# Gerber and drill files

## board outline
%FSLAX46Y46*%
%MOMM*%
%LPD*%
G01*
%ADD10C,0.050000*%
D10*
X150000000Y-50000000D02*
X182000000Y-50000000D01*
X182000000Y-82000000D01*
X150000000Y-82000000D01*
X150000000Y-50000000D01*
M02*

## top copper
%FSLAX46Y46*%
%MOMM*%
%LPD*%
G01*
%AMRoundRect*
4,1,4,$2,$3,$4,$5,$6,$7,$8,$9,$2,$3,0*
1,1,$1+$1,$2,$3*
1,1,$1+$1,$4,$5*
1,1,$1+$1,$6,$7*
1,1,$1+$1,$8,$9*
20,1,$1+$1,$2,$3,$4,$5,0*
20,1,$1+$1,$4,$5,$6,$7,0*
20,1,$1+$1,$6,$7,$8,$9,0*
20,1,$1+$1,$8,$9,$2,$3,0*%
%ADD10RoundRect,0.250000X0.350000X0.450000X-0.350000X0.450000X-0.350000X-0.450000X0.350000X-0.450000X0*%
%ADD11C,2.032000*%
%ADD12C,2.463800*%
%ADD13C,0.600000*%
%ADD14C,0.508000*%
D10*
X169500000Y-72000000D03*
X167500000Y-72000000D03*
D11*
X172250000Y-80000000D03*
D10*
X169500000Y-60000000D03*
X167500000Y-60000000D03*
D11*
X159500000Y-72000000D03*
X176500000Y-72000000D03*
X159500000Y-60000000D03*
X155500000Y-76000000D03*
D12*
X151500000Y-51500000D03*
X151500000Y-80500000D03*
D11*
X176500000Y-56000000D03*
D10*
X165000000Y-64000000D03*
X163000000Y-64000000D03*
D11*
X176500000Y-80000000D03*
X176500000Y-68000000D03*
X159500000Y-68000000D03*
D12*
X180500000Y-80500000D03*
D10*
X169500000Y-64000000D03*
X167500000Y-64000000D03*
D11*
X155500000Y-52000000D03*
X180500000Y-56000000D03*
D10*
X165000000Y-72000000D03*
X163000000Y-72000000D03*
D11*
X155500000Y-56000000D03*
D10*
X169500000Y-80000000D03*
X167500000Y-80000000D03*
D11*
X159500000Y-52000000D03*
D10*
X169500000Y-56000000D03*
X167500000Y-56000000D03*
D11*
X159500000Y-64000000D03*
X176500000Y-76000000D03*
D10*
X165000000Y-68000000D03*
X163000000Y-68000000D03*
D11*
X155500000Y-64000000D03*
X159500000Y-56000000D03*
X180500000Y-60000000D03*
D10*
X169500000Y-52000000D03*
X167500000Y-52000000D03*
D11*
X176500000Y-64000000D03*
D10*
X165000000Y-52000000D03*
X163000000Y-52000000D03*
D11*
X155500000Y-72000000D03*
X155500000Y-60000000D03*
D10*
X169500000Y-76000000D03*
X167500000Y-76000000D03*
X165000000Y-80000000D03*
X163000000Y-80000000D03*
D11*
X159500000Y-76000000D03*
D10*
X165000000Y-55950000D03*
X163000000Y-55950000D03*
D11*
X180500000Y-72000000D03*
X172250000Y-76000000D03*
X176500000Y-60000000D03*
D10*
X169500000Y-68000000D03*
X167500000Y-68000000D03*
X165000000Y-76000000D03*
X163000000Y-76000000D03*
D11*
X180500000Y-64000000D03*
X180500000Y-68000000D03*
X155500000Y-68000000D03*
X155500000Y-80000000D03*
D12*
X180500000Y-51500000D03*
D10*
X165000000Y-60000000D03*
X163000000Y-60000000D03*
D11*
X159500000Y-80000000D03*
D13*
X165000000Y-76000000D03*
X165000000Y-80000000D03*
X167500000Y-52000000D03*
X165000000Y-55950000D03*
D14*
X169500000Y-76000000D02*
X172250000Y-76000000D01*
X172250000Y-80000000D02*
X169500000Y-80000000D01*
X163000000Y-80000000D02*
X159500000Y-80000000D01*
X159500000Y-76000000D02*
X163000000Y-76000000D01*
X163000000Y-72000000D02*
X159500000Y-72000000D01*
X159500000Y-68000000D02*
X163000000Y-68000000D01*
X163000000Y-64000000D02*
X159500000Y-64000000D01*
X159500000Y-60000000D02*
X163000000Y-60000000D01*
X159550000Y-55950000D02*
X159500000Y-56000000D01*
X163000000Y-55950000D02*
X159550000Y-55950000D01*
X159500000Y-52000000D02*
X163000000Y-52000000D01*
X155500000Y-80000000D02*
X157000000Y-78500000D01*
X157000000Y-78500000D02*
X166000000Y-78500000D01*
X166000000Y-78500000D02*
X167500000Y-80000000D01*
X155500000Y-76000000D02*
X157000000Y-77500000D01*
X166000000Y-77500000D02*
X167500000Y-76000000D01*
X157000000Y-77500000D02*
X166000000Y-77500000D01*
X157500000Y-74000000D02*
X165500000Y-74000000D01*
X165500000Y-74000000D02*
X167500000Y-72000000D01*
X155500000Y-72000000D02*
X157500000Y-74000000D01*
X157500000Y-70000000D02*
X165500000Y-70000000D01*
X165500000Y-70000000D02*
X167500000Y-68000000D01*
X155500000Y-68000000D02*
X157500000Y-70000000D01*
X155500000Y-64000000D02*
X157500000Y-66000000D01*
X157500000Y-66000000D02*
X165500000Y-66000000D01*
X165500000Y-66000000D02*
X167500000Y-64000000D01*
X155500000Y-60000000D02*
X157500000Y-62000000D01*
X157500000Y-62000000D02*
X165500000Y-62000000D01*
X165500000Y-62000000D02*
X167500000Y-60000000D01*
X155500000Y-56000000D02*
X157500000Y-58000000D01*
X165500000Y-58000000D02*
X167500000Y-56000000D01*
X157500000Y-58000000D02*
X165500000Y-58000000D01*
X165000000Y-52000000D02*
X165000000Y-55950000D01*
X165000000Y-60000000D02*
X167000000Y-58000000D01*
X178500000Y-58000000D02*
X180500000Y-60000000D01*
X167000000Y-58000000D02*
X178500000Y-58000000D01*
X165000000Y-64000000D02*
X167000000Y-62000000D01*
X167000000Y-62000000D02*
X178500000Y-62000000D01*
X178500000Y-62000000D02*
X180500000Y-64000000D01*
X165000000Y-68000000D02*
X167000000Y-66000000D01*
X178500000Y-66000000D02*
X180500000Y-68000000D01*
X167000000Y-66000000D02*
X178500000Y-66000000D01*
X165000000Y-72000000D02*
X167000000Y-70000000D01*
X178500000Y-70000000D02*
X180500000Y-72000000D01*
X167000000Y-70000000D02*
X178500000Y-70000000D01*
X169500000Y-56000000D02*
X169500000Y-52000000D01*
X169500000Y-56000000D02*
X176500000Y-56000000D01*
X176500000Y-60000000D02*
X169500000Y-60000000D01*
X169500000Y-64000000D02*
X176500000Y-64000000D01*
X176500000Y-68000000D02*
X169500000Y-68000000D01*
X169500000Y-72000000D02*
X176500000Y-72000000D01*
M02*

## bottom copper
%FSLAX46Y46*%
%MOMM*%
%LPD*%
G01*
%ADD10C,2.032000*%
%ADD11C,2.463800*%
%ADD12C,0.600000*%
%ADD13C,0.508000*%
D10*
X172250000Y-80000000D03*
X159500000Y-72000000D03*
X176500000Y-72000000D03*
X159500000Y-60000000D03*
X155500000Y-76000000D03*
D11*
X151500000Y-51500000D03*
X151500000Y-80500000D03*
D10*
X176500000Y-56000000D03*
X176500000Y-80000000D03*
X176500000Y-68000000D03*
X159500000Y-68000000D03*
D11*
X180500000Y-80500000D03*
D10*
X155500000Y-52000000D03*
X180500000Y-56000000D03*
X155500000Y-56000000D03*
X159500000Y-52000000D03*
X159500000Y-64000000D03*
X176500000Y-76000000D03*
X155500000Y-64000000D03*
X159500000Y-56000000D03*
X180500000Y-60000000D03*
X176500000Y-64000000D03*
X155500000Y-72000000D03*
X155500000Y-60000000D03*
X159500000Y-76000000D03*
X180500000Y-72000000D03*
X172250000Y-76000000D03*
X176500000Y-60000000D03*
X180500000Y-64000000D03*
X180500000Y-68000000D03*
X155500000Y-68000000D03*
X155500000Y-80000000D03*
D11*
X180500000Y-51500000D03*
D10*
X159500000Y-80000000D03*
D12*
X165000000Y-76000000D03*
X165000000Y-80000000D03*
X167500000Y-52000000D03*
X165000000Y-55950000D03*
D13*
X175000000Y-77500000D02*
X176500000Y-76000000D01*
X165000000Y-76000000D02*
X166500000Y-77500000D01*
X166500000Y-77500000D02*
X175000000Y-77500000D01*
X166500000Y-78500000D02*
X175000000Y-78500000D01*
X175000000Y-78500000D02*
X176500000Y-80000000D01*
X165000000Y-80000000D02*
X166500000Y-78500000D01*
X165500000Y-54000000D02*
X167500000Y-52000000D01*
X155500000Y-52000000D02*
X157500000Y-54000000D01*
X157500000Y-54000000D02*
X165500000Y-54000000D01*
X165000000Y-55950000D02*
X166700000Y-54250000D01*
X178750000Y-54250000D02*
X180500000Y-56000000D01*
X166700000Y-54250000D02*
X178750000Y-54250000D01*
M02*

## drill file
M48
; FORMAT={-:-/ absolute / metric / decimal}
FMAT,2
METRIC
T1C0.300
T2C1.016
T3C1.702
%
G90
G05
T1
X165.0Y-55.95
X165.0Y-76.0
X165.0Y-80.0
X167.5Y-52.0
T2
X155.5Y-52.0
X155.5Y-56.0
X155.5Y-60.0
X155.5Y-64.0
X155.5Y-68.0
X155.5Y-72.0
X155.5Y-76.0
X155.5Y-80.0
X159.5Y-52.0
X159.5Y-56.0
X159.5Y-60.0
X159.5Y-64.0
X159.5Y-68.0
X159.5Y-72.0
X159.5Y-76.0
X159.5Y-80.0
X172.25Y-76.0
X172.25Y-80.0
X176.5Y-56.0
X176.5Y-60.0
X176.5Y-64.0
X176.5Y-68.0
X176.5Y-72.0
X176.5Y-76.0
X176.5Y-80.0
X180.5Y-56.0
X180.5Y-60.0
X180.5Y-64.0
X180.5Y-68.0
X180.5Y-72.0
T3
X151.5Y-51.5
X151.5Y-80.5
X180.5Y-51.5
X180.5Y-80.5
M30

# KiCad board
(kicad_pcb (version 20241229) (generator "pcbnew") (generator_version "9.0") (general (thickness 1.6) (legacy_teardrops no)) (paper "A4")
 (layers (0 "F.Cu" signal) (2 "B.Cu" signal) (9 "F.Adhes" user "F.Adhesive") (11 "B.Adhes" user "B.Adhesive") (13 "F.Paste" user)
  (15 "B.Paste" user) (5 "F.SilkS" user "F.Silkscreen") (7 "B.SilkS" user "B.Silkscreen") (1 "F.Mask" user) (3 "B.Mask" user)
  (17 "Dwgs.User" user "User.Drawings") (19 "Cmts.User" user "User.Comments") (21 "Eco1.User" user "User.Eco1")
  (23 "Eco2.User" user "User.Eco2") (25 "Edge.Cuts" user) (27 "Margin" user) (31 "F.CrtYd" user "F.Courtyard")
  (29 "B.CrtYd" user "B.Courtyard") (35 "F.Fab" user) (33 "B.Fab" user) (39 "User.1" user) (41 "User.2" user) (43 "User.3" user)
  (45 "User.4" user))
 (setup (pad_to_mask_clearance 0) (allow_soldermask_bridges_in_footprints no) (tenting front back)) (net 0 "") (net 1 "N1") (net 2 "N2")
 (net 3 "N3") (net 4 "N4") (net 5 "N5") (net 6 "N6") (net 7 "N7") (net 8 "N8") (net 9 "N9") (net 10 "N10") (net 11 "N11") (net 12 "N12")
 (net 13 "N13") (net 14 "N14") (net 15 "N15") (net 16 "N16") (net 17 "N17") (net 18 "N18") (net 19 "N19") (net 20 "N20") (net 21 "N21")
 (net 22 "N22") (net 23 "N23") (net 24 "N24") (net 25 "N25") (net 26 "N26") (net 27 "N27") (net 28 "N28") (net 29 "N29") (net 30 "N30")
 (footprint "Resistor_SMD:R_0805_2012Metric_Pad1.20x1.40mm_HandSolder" (layer "F.Cu") (at 168.5 72 180)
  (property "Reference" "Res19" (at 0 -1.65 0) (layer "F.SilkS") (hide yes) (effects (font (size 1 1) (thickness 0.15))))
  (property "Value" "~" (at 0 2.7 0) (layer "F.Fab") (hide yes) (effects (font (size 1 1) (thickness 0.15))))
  (pad "1" smd roundrect (at -1 0 180) (size 1.2 1.4) (layers "F.Cu" "F.Mask" "F.Paste") (roundrect_rratio 0.208333) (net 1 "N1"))
  (pad "2" smd roundrect (at 1 0 180) (size 1.2 1.4) (layers "F.Cu" "F.Mask" "F.Paste") (roundrect_rratio 0.208333) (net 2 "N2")))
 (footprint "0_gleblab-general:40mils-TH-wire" (layer "F.Cu") (at 172.25 80)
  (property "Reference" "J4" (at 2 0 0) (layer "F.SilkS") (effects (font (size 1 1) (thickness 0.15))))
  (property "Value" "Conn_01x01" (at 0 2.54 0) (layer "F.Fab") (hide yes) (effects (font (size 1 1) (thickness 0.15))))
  (pad "1" thru_hole circle (at 0 0) (size 2.032 2.032) (drill 1.016) (layers "*.Cu" "*.Mask") (remove_unused_layers no) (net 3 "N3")))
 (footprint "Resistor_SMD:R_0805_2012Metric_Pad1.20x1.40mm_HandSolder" (layer "F.Cu") (at 168.5 60 180)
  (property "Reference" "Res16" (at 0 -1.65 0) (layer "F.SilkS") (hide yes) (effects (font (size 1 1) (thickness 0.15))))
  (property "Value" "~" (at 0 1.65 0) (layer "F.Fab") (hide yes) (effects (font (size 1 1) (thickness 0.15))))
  (pad "1" smd roundrect (at -1 0 180) (size 1.2 1.4) (layers "F.Cu" "F.Mask" "F.Paste") (roundrect_rratio 0.208333) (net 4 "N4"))
  (pad "2" smd roundrect (at 1 0 180) (size 1.2 1.4) (layers "F.Cu" "F.Mask" "F.Paste") (roundrect_rratio 0.208333) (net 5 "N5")))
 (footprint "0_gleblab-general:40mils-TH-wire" (layer "F.Cu") (at 159.5 72 180)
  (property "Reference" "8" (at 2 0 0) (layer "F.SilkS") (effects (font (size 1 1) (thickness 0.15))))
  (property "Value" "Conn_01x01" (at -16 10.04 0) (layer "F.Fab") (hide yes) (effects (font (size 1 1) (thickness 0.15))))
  (pad "1" thru_hole circle (at 0 0 180) (size 2.032 2.032) (drill 1.016) (layers "*.Cu" "*.Mask") (remove_unused_layers no) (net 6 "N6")))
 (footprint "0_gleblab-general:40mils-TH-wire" (layer "F.Cu") (at 176.5 72)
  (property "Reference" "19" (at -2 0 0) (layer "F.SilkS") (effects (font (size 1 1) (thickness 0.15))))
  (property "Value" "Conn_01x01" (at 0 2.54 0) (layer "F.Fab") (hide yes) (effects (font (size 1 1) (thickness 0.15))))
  (pad "1" thru_hole circle (at 0 0) (size 2.032 2.032) (drill 1.016) (layers "*.Cu" "*.Mask") (remove_unused_layers no) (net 1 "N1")))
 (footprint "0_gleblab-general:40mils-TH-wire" (layer "F.Cu") (at 159.5 60 180)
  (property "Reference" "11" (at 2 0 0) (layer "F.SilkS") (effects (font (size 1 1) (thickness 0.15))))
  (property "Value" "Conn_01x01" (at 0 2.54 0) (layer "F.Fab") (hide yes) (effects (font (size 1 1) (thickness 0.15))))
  (pad "1" thru_hole circle (at 0 0 180) (size 2.032 2.032) (drill 1.016) (layers "*.Cu" "*.Mask") (remove_unused_layers no) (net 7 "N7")))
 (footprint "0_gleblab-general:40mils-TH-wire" (layer "F.Cu") (at 155.5 76 180)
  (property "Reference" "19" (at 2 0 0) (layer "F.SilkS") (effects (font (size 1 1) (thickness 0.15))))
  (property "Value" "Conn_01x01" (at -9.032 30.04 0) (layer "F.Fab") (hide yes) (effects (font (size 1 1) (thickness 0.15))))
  (pad "1" thru_hole circle (at 0 0 180) (size 2.032 2.032) (drill 1.016) (layers "*.Cu" "*.Mask") (remove_unused_layers no) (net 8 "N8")))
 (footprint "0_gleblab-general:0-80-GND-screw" (layer "F.Cu") (at 151.5 51.5)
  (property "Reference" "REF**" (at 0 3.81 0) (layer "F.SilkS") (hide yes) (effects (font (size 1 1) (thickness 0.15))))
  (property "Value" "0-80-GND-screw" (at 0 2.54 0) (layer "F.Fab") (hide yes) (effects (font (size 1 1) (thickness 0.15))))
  (pad "1" thru_hole circle (at 0 0) (size 2.4638 2.4638) (drill 1.7018) (layers "*.Cu" "*.Mask") (remove_unused_layers no)))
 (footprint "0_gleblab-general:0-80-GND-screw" (layer "F.Cu") (at 151.5 80.5)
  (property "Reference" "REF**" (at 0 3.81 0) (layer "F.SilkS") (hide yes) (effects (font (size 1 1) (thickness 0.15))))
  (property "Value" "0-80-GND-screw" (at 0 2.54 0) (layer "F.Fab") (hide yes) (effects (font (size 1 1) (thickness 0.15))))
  (pad "1" thru_hole circle (at 0 0) (size 2.4638 2.4638) (drill 1.7018) (layers "*.Cu" "*.Mask") (remove_unused_layers no)))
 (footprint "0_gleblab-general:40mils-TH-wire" (layer "F.Cu") (at 176.5 56)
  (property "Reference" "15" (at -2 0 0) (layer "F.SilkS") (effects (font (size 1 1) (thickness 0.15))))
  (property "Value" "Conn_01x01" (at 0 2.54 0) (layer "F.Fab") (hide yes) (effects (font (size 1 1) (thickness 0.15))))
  (pad "1" thru_hole circle (at 0 0) (size 2.032 2.032) (drill 1.016) (layers "*.Cu" "*.Mask") (remove_unused_layers no) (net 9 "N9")))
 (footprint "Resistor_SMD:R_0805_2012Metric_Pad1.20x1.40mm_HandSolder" (layer "F.Cu") (at 164 64 180)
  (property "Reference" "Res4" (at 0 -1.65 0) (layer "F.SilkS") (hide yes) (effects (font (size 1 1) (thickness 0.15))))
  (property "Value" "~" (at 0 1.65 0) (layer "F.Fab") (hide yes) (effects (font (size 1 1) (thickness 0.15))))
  (pad "1" smd roundrect (at -1 0 180) (size 1.2 1.4) (layers "F.Cu" "F.Mask" "F.Paste") (roundrect_rratio 0.208333) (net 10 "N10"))
  (pad "2" smd roundrect (at 1 0 180) (size 1.2 1.4) (layers "F.Cu" "F.Mask" "F.Paste") (roundrect_rratio 0.208333) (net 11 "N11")))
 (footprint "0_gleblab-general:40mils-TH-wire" (layer "F.Cu") (at 176.5 80)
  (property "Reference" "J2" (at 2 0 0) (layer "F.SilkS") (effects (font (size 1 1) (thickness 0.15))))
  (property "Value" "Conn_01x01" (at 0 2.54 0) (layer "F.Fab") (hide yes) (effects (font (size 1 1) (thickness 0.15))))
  (pad "1" thru_hole circle (at 0 0) (size 2.032 2.032) (drill 1.016) (layers "*.Cu" "*.Mask") (remove_unused_layers no) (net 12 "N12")))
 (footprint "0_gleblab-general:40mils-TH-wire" (layer "F.Cu") (at 176.5 68)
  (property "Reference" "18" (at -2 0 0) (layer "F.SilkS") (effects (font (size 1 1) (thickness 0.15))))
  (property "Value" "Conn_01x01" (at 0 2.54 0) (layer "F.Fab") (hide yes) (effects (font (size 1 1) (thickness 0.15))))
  (pad "1" thru_hole circle (at 0 0) (size 2.032 2.032) (drill 1.016) (layers "*.Cu" "*.Mask") (remove_unused_layers no) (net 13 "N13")))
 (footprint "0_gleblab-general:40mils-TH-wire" (layer "F.Cu") (at 159.5 68 180)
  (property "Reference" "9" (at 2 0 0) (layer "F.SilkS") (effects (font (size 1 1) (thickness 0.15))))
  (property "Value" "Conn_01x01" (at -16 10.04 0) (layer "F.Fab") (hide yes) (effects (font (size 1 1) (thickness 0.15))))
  (pad "1" thru_hole circle (at 0 0 180) (size 2.032 2.032) (drill 1.016) (layers "*.Cu" "*.Mask") (remove_unused_layers no) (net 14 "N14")))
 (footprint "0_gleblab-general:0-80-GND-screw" (layer "F.Cu") (at 180.5 80.5)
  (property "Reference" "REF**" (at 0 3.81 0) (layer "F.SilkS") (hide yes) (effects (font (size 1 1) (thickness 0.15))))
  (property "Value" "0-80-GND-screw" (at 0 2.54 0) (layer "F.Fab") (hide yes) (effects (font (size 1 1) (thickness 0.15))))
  (pad "1" thru_hole circle (at 0 0) (size 2.4638 2.4638) (drill 1.7018) (layers "*.Cu" "*.Mask") (remove_unused_layers no)))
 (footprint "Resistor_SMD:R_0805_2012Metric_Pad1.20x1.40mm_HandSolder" (layer "F.Cu") (at 168.5 64 180)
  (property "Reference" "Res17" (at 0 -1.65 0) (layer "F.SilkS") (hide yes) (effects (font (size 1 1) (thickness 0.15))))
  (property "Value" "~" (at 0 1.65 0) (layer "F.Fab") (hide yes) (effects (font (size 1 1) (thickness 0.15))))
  (pad "1" smd roundrect (at -1 0 180) (size 1.2 1.4) (layers "F.Cu" "F.Mask" "F.Paste") (roundrect_rratio 0.208333) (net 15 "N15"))
  (pad "2" smd roundrect (at 1 0 180) (size 1.2 1.4) (layers "F.Cu" "F.Mask" "F.Paste") (roundrect_rratio 0.208333) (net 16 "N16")))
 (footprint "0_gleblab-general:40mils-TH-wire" (layer "F.Cu") (at 155.5 52 180)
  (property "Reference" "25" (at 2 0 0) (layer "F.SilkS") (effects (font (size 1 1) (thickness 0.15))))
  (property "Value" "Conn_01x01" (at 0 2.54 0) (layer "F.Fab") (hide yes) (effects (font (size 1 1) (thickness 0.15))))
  (pad "1" thru_hole circle (at 0 0 180) (size 2.032 2.032) (drill 1.016) (layers "*.Cu" "*.Mask") (remove_unused_layers no) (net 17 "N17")))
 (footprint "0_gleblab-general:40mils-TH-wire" (layer "F.Cu") (at 180.5 56)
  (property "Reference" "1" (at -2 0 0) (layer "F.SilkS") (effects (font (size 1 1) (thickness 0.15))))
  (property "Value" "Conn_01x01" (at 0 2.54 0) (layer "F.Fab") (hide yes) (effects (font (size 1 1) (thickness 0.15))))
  (pad "1" thru_hole circle (at 0 0) (size 2.032 2.032) (drill 1.016) (layers "*.Cu" "*.Mask") (remove_unused_layers no) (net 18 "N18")))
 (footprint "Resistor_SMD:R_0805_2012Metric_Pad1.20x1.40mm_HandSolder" (layer "F.Cu") (at 164 72 180)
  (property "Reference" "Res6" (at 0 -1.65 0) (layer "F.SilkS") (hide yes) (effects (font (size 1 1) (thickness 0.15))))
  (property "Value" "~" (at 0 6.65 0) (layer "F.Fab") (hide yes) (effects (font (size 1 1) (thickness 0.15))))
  (pad "1" smd roundrect (at -1 0 180) (size 1.2 1.4) (layers "F.Cu" "F.Mask" "F.Paste") (roundrect_rratio 0.208333) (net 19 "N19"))
  (pad "2" smd roundrect (at 1 0 180) (size 1.2 1.4) (layers "F.Cu" "F.Mask" "F.Paste") (roundrect_rratio 0.208333) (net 6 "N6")))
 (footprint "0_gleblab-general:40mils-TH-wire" (layer "F.Cu") (at 155.5 56 180)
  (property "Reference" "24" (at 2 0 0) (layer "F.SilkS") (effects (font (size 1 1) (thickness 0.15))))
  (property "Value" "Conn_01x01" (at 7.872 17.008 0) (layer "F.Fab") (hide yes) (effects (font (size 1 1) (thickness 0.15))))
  (pad "1" thru_hole circle (at 0 0 180) (size 2.032 2.032) (drill 1.016) (layers "*.Cu" "*.Mask") (remove_unused_layers no) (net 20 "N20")))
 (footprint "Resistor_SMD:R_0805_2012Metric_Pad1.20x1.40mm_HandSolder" (layer "F.Cu") (at 168.5 80 180)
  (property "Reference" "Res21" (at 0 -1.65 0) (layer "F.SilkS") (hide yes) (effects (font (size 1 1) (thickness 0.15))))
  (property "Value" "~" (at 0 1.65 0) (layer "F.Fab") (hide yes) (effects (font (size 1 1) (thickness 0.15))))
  (pad "1" smd roundrect (at -1 0 180) (size 1.2 1.4) (layers "F.Cu" "F.Mask" "F.Paste") (roundrect_rratio 0.208333) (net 3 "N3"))
  (pad "2" smd roundrect (at 1 0 180) (size 1.2 1.4) (layers "F.Cu" "F.Mask" "F.Paste") (roundrect_rratio 0.208333) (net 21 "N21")))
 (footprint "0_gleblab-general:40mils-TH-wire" (layer "F.Cu") (at 159.5 52 180)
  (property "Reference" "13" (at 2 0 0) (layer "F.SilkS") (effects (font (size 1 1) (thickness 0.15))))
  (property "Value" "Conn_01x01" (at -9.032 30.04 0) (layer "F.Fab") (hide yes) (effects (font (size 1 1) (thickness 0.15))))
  (pad "1" thru_hole circle (at 0 0 180) (size 2.032 2.032) (drill 1.016) (layers "*.Cu" "*.Mask") (remove_unused_layers no) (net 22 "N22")))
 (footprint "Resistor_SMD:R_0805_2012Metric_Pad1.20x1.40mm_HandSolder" (layer "F.Cu") (at 168.5 56 180)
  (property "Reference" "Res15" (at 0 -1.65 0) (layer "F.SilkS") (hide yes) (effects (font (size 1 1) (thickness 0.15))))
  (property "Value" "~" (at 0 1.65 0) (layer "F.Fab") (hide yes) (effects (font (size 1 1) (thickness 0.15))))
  (pad "1" smd roundrect (at -1 0 180) (size 1.2 1.4) (layers "F.Cu" "F.Mask" "F.Paste") (roundrect_rratio 0.208333) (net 9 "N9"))
  (pad "2" smd roundrect (at 1 0 180) (size 1.2 1.4) (layers "F.Cu" "F.Mask" "F.Paste") (roundrect_rratio 0.208333) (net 20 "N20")))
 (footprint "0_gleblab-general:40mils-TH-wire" (layer "F.Cu") (at 159.5 64 180)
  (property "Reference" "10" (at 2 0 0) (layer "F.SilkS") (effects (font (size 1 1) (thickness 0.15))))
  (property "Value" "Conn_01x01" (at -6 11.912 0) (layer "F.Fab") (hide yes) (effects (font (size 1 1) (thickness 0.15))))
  (pad "1" thru_hole circle (at 0 0 180) (size 2.032 2.032) (drill 1.016) (layers "*.Cu" "*.Mask") (remove_unused_layers no) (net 11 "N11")))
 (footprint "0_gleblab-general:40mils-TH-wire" (layer "F.Cu") (at 176.5 76)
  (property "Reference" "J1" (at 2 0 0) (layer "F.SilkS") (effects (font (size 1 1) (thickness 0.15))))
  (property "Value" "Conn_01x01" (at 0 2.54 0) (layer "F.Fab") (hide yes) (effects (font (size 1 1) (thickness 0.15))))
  (pad "1" thru_hole circle (at 0 0) (size 2.032 2.032) (drill 1.016) (layers "*.Cu" "*.Mask") (remove_unused_layers no) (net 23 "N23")))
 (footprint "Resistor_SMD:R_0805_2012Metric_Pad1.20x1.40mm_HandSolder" (layer "F.Cu") (at 164 68 180)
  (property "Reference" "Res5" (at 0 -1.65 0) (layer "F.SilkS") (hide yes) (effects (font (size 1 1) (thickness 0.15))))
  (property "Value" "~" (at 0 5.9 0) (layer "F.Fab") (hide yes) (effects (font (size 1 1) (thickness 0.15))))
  (pad "1" smd roundrect (at -1 0 180) (size 1.2 1.4) (layers "F.Cu" "F.Mask" "F.Paste") (roundrect_rratio 0.208333) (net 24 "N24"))
  (pad "2" smd roundrect (at 1 0 180) (size 1.2 1.4) (layers "F.Cu" "F.Mask" "F.Paste") (roundrect_rratio 0.208333) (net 14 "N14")))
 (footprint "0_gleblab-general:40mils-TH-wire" (layer "F.Cu") (at 155.5 64 180)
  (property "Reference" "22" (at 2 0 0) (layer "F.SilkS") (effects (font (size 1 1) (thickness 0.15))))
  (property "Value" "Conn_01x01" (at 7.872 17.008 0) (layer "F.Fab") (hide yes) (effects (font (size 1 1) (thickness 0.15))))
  (pad "1" thru_hole circle (at 0 0 180) (size 2.032 2.032) (drill 1.016) (layers "*.Cu" "*.Mask") (remove_unused_layers no) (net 16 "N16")))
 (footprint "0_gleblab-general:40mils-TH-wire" (layer "F.Cu") (at 159.5 56 180)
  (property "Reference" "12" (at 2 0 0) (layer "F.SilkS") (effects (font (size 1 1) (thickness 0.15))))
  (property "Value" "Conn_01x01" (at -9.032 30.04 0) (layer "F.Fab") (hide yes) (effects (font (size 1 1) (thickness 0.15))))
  (pad "1" thru_hole circle (at 0 0 180) (size 2.032 2.032) (drill 1.016) (layers "*.Cu" "*.Mask") (remove_unused_layers no) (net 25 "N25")))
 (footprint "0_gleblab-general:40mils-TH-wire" (layer "F.Cu") (at 180.5 60)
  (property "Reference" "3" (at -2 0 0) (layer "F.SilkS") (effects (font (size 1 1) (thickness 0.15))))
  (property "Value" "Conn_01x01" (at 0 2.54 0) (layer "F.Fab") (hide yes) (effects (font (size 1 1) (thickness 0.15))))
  (pad "1" thru_hole circle (at 0 0) (size 2.032 2.032) (drill 1.016) (layers "*.Cu" "*.Mask") (remove_unused_layers no) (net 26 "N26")))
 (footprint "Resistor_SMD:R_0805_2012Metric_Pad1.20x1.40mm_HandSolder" (layer "F.Cu") (at 168.5 52 180)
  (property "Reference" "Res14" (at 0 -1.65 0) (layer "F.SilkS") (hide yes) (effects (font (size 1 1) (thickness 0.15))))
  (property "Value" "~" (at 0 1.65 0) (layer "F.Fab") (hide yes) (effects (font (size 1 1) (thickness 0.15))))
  (pad "1" smd roundrect (at -1 0 180) (size 1.2 1.4) (layers "F.Cu" "F.Mask" "F.Paste") (roundrect_rratio 0.208333) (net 9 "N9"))
  (pad "2" smd roundrect (at 1 0 180) (size 1.2 1.4) (layers "F.Cu" "F.Mask" "F.Paste") (roundrect_rratio 0.208333) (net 17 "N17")))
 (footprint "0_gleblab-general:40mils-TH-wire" (layer "F.Cu") (at 176.5 64)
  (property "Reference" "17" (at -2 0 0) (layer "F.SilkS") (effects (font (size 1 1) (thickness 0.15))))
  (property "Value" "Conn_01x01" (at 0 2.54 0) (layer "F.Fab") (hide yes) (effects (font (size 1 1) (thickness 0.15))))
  (pad "1" thru_hole circle (at 0 0) (size 2.032 2.032) (drill 1.016) (layers "*.Cu" "*.Mask") (remove_unused_layers no) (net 15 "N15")))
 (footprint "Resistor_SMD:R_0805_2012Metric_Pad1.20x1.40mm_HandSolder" (layer "F.Cu") (at 164 52 180)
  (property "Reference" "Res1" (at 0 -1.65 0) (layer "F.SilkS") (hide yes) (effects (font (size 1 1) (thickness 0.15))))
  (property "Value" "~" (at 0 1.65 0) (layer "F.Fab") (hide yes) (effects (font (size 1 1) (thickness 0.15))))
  (pad "1" smd roundrect (at -1 0 180) (size 1.2 1.4) (layers "F.Cu" "F.Mask" "F.Paste") (roundrect_rratio 0.208333) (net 18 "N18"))
  (pad "2" smd roundrect (at 1 0 180) (size 1.2 1.4) (layers "F.Cu" "F.Mask" "F.Paste") (roundrect_rratio 0.208333) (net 22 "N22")))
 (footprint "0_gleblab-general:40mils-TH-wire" (layer "F.Cu") (at 155.5 72 180)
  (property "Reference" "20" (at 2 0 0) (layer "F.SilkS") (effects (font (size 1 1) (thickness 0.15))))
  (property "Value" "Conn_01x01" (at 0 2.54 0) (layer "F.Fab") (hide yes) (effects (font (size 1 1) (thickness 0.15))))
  (pad "1" thru_hole circle (at 0 0 180) (size 2.032 2.032) (drill 1.016) (layers "*.Cu" "*.Mask") (remove_unused_layers no) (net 2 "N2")))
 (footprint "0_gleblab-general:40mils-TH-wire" (layer "F.Cu") (at 155.5 60 180)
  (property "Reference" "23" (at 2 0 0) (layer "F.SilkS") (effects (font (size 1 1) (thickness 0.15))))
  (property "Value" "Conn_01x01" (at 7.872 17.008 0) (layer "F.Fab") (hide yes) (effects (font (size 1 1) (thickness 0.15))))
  (pad "1" thru_hole circle (at 0 0 180) (size 2.032 2.032) (drill 1.016) (layers "*.Cu" "*.Mask") (remove_unused_layers no) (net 5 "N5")))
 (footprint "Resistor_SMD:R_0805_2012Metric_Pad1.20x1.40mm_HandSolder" (layer "F.Cu") (at 168.5 76 180)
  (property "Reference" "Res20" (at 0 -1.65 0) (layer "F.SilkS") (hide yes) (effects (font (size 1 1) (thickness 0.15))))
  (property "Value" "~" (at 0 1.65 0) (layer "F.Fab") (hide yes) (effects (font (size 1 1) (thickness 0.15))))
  (pad "1" smd roundrect (at -1 0 180) (size 1.2 1.4) (layers "F.Cu" "F.Mask" "F.Paste") (roundrect_rratio 0.208333) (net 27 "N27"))
  (pad "2" smd roundrect (at 1 0 180) (size 1.2 1.4) (layers "F.Cu" "F.Mask" "F.Paste") (roundrect_rratio 0.208333) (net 8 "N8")))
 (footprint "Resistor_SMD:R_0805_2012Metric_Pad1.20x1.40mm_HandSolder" (layer "F.Cu") (at 164 80 180)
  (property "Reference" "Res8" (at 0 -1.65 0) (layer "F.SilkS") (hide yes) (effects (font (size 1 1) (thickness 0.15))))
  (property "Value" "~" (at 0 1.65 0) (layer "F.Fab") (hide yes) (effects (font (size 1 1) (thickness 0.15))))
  (pad "1" smd roundrect (at -1 0 180) (size 1.2 1.4) (layers "F.Cu" "F.Mask" "F.Paste") (roundrect_rratio 0.208333) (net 12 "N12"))
  (pad "2" smd roundrect (at 1 0 180) (size 1.2 1.4) (layers "F.Cu" "F.Mask" "F.Paste") (roundrect_rratio 0.208333) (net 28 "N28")))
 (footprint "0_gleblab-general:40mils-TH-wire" (layer "F.Cu") (at 159.5 76 180)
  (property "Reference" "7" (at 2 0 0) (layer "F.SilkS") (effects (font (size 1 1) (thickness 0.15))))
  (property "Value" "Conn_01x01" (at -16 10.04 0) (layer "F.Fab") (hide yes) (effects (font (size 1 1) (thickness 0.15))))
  (pad "1" thru_hole circle (at 0 0 180) (size 2.032 2.032) (drill 1.016) (layers "*.Cu" "*.Mask") (remove_unused_layers no) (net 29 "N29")))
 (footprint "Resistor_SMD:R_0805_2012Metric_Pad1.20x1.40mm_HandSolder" (layer "F.Cu") (at 164 55.95 180)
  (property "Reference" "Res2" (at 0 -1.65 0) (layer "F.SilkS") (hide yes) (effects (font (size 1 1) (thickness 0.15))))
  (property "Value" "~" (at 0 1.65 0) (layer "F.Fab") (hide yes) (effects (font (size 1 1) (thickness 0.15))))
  (pad "1" smd roundrect (at -1 0 180) (size 1.2 1.4) (layers "F.Cu" "F.Mask" "F.Paste") (roundrect_rratio 0.208333) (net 18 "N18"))
  (pad "2" smd roundrect (at 1 0 180) (size 1.2 1.4) (layers "F.Cu" "F.Mask" "F.Paste") (roundrect_rratio 0.208333) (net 25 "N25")))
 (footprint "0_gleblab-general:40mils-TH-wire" (layer "F.Cu") (at 180.5 72)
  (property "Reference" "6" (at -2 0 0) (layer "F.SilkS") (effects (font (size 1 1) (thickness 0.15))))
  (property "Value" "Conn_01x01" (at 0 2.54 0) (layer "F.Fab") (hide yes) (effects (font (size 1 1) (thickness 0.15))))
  (pad "1" thru_hole circle (at 0 0) (size 2.032 2.032) (drill 1.016) (layers "*.Cu" "*.Mask") (remove_unused_layers no) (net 19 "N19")))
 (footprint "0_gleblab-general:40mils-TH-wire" (layer "F.Cu") (at 172.25 76)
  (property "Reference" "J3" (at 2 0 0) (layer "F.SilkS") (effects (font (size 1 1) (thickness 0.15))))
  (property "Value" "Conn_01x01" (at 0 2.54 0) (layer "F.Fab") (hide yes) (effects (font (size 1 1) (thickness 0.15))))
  (pad "1" thru_hole circle (at 0 0) (size 2.032 2.032) (drill 1.016) (layers "*.Cu" "*.Mask") (remove_unused_layers no) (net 27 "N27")))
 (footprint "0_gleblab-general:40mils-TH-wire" (layer "F.Cu") (at 176.5 60)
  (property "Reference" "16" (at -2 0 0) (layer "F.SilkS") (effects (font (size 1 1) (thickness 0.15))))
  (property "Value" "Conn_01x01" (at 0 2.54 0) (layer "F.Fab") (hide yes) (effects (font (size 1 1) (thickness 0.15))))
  (pad "1" thru_hole circle (at 0 0) (size 2.032 2.032) (drill 1.016) (layers "*.Cu" "*.Mask") (remove_unused_layers no) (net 4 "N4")))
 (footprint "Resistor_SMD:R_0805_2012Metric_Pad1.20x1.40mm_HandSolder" (layer "F.Cu") (at 168.5 68 180)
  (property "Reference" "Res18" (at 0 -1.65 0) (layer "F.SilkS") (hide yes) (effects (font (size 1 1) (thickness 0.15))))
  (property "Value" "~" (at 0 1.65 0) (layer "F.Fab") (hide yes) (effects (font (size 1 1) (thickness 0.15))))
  (pad "1" smd roundrect (at -1 0 180) (size 1.2 1.4) (layers "F.Cu" "F.Mask" "F.Paste") (roundrect_rratio 0.208333) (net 13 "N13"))
  (pad "2" smd roundrect (at 1 0 180) (size 1.2 1.4) (layers "F.Cu" "F.Mask" "F.Paste") (roundrect_rratio 0.208333) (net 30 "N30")))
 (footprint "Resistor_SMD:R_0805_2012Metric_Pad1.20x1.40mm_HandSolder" (layer "F.Cu") (at 164 76 180)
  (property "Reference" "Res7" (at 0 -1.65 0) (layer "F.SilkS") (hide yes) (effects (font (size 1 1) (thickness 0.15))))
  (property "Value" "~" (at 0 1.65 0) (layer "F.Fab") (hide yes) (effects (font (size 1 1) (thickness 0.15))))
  (pad "1" smd roundrect (at -1 0 180) (size 1.2 1.4) (layers "F.Cu" "F.Mask" "F.Paste") (roundrect_rratio 0.208333) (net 23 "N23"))
  (pad "2" smd roundrect (at 1 0 180) (size 1.2 1.4) (layers "F.Cu" "F.Mask" "F.Paste") (roundrect_rratio 0.208333) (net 29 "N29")))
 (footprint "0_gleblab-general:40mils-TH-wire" (layer "F.Cu") (at 180.5 64)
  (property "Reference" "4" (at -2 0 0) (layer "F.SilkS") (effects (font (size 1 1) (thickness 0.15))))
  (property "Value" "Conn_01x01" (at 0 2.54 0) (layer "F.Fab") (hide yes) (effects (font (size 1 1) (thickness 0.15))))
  (pad "1" thru_hole circle (at 0 0) (size 2.032 2.032) (drill 1.016) (layers "*.Cu" "*.Mask") (remove_unused_layers no) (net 10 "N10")))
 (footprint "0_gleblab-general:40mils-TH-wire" (layer "F.Cu") (at 180.5 68)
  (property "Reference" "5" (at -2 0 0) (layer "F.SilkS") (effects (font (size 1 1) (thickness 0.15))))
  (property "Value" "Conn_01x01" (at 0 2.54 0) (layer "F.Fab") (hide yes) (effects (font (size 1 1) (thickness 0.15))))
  (pad "1" thru_hole circle (at 0 0) (size 2.032 2.032) (drill 1.016) (layers "*.Cu" "*.Mask") (remove_unused_layers no) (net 24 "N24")))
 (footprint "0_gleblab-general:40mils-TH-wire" (layer "F.Cu") (at 155.5 68 180)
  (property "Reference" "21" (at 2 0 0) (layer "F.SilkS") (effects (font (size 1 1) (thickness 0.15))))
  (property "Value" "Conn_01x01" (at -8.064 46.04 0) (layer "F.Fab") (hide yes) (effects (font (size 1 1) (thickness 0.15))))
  (pad "1" thru_hole circle (at 0 0 180) (size 2.032 2.032) (drill 1.016) (layers "*.Cu" "*.Mask") (remove_unused_layers no) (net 30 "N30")))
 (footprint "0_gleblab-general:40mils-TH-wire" (layer "F.Cu") (at 155.5 80 180)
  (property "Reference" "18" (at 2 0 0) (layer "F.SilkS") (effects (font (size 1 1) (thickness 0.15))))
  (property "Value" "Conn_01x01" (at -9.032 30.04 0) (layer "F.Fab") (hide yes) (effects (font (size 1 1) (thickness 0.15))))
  (pad "1" thru_hole circle (at 0 0 180) (size 2.032 2.032) (drill 1.016) (layers "*.Cu" "*.Mask") (remove_unused_layers no) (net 21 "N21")))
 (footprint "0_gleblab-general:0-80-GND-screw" (layer "F.Cu") (at 180.5 51.5)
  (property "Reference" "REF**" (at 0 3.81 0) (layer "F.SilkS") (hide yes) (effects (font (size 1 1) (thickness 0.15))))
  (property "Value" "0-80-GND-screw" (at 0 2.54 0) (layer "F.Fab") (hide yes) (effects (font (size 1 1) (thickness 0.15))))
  (pad "1" thru_hole circle (at 0 0) (size 2.4638 2.4638) (drill 1.7018) (layers "*.Cu" "*.Mask") (remove_unused_layers no)))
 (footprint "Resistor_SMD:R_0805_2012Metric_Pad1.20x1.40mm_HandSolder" (layer "F.Cu") (at 164 60 180)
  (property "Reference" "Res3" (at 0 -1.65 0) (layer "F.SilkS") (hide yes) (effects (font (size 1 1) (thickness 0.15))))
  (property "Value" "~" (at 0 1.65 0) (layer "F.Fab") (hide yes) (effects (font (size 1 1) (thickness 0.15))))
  (pad "1" smd roundrect (at -1 0 180) (size 1.2 1.4) (layers "F.Cu" "F.Mask" "F.Paste") (roundrect_rratio 0.208333) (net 26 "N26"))
  (pad "2" smd roundrect (at 1 0 180) (size 1.2 1.4) (layers "F.Cu" "F.Mask" "F.Paste") (roundrect_rratio 0.208333) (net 7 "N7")))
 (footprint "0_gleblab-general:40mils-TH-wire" (layer "F.Cu") (at 159.5 80 180)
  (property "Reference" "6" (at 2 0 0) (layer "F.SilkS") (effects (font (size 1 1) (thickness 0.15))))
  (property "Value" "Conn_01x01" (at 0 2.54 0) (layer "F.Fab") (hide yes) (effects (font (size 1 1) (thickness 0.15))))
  (pad "1" thru_hole circle (at 0 0 180) (size 2.032 2.032) (drill 1.016) (layers "*.Cu" "*.Mask") (remove_unused_layers no) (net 28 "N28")))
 (gr_rect (start 150 50) (end 182 82) (stroke (width 0.05) (type default)) (fill no) (layer "Edge.Cuts"))
 (via (at 165 76) (size 0.6) (drill 0.3) (layers "F.Cu" "B.Cu") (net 23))
 (segment (start 175 77.5) (end 176.5 76) (width 0.508) (layer "B.Cu") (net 23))
 (segment (start 165 76) (end 166.5 77.5) (width 0.508) (layer "B.Cu") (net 23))
 (segment (start 166.5 77.5) (end 175 77.5) (width 0.508) (layer "B.Cu") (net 23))
 (via (at 165 80) (size 0.6) (drill 0.3) (layers "F.Cu" "B.Cu") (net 12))
 (segment (start 166.5 78.5) (end 175 78.5) (width 0.508) (layer "B.Cu") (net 12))
 (segment (start 175 78.5) (end 176.5 80) (width 0.508) (layer "B.Cu") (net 12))
 (segment (start 165 80) (end 166.5 78.5) (width 0.508) (layer "B.Cu") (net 12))
 (segment (start 169.5 76) (end 172.25 76) (width 0.508) (layer "F.Cu") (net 27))
 (segment (start 172.25 80) (end 169.5 80) (width 0.508) (layer "F.Cu") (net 3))
 (segment (start 163 80) (end 159.5 80) (width 0.508) (layer "F.Cu") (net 28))
 (segment (start 159.5 76) (end 163 76) (width 0.508) (layer "F.Cu") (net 29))
 (segment (start 163 72) (end 159.5 72) (width 0.508) (layer "F.Cu") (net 6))
 (segment (start 159.5 68) (end 163 68) (width 0.508) (layer "F.Cu") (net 14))
 (segment (start 163 64) (end 159.5 64) (width 0.508) (layer "F.Cu") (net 11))
 (segment (start 159.5 60) (end 163 60) (width 0.508) (layer "F.Cu") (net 7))
 (segment (start 159.55 55.95) (end 159.5 56) (width 0.508) (layer "F.Cu") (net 25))
 (segment (start 163 55.95) (end 159.55 55.95) (width 0.508) (layer "F.Cu") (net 25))
 (segment (start 159.5 52) (end 163 52) (width 0.508) (layer "F.Cu") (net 22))
 (segment (start 155.5 80) (end 157 78.5) (width 0.508) (layer "F.Cu") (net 21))
 (segment (start 157 78.5) (end 166 78.5) (width 0.508) (layer "F.Cu") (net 21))
 (segment (start 166 78.5) (end 167.5 80) (width 0.508) (layer "F.Cu") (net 21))
 (segment (start 155.5 76) (end 157 77.5) (width 0.508) (layer "F.Cu") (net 8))
 (segment (start 166 77.5) (end 167.5 76) (width 0.508) (layer "F.Cu") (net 8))
 (segment (start 157 77.5) (end 166 77.5) (width 0.508) (layer "F.Cu") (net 8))
 (segment (start 157.5 74) (end 165.5 74) (width 0.508) (layer "F.Cu") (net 2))
 (segment (start 165.5 74) (end 167.5 72) (width 0.508) (layer "F.Cu") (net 2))
 (segment (start 155.5 72) (end 157.5 74) (width 0.508) (layer "F.Cu") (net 2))
 (segment (start 157.5 70) (end 165.5 70) (width 0.508) (layer "F.Cu") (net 30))
 (segment (start 165.5 70) (end 167.5 68) (width 0.508) (layer "F.Cu") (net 30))
 (segment (start 155.5 68) (end 157.5 70) (width 0.508) (layer "F.Cu") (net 30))
 (segment (start 155.5 64) (end 157.5 66) (width 0.508) (layer "F.Cu") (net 16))
 (segment (start 157.5 66) (end 165.5 66) (width 0.508) (layer "F.Cu") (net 16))
 (segment (start 165.5 66) (end 167.5 64) (width 0.508) (layer "F.Cu") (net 16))
 (segment (start 155.5 60) (end 157.5 62) (width 0.508) (layer "F.Cu") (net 5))
 (segment (start 157.5 62) (end 165.5 62) (width 0.508) (layer "F.Cu") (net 5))
 (segment (start 165.5 62) (end 167.5 60) (width 0.508) (layer "F.Cu") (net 5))
 (segment (start 155.5 56) (end 157.5 58) (width 0.508) (layer "F.Cu") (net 20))
 (segment (start 165.5 58) (end 167.5 56) (width 0.508) (layer "F.Cu") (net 20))
 (segment (start 157.5 58) (end 165.5 58) (width 0.508) (layer "F.Cu") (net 20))
 (via (at 167.5 52) (size 0.6) (drill 0.3) (layers "F.Cu" "B.Cu") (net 17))
 (segment (start 165.5 54) (end 167.5 52) (width 0.508) (layer "B.Cu") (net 17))
 (segment (start 155.5 52) (end 157.5 54) (width 0.508) (layer "B.Cu") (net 17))
 (segment (start 157.5 54) (end 165.5 54) (width 0.508) (layer "B.Cu") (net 17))
 (segment (start 165 52) (end 165 55.95) (width 0.508) (layer "F.Cu") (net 18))
 (via (at 165 55.95) (size 0.6) (drill 0.3) (layers "F.Cu" "B.Cu") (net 18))
 (segment (start 165 55.95) (end 166.7 54.25) (width 0.508) (layer "B.Cu") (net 18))
 (segment (start 178.75 54.25) (end 180.5 56) (width 0.508) (layer "B.Cu") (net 18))
 (segment (start 166.7 54.25) (end 178.75 54.25) (width 0.508) (layer "B.Cu") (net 18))
 (segment (start 165 60) (end 167 58) (width 0.508) (layer "F.Cu") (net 26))
 (segment (start 178.5 58) (end 180.5 60) (width 0.508) (layer "F.Cu") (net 26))
 (segment (start 167 58) (end 178.5 58) (width 0.508) (layer "F.Cu") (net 26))
 (segment (start 165 64) (end 167 62) (width 0.508) (layer "F.Cu") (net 10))
 (segment (start 167 62) (end 178.5 62) (width 0.508) (layer "F.Cu") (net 10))
 (segment (start 178.5 62) (end 180.5 64) (width 0.508) (layer "F.Cu") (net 10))
 (segment (start 165 68) (end 167 66) (width 0.508) (layer "F.Cu") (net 24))
 (segment (start 178.5 66) (end 180.5 68) (width 0.508) (layer "F.Cu") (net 24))
 (segment (start 167 66) (end 178.5 66) (width 0.508) (layer "F.Cu") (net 24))
 (segment (start 165 72) (end 167 70) (width 0.508) (layer "F.Cu") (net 19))
 (segment (start 178.5 70) (end 180.5 72) (width 0.508) (layer "F.Cu") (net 19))
 (segment (start 167 70) (end 178.5 70) (width 0.508) (layer "F.Cu") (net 19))
 (segment (start 169.5 56) (end 169.5 52) (width 0.508) (layer "F.Cu") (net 9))
 (segment (start 169.5 56) (end 176.5 56) (width 0.508) (layer "F.Cu") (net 9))
 (segment (start 176.5 60) (end 169.5 60) (width 0.508) (layer "F.Cu") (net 4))
 (segment (start 169.5 64) (end 176.5 64) (width 0.508) (layer "F.Cu") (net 15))
 (segment (start 176.5 68) (end 169.5 68) (width 0.508) (layer "F.Cu") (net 13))
 (segment (start 169.5 72) (end 176.5 72) (width 0.508) (layer "F.Cu") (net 1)))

